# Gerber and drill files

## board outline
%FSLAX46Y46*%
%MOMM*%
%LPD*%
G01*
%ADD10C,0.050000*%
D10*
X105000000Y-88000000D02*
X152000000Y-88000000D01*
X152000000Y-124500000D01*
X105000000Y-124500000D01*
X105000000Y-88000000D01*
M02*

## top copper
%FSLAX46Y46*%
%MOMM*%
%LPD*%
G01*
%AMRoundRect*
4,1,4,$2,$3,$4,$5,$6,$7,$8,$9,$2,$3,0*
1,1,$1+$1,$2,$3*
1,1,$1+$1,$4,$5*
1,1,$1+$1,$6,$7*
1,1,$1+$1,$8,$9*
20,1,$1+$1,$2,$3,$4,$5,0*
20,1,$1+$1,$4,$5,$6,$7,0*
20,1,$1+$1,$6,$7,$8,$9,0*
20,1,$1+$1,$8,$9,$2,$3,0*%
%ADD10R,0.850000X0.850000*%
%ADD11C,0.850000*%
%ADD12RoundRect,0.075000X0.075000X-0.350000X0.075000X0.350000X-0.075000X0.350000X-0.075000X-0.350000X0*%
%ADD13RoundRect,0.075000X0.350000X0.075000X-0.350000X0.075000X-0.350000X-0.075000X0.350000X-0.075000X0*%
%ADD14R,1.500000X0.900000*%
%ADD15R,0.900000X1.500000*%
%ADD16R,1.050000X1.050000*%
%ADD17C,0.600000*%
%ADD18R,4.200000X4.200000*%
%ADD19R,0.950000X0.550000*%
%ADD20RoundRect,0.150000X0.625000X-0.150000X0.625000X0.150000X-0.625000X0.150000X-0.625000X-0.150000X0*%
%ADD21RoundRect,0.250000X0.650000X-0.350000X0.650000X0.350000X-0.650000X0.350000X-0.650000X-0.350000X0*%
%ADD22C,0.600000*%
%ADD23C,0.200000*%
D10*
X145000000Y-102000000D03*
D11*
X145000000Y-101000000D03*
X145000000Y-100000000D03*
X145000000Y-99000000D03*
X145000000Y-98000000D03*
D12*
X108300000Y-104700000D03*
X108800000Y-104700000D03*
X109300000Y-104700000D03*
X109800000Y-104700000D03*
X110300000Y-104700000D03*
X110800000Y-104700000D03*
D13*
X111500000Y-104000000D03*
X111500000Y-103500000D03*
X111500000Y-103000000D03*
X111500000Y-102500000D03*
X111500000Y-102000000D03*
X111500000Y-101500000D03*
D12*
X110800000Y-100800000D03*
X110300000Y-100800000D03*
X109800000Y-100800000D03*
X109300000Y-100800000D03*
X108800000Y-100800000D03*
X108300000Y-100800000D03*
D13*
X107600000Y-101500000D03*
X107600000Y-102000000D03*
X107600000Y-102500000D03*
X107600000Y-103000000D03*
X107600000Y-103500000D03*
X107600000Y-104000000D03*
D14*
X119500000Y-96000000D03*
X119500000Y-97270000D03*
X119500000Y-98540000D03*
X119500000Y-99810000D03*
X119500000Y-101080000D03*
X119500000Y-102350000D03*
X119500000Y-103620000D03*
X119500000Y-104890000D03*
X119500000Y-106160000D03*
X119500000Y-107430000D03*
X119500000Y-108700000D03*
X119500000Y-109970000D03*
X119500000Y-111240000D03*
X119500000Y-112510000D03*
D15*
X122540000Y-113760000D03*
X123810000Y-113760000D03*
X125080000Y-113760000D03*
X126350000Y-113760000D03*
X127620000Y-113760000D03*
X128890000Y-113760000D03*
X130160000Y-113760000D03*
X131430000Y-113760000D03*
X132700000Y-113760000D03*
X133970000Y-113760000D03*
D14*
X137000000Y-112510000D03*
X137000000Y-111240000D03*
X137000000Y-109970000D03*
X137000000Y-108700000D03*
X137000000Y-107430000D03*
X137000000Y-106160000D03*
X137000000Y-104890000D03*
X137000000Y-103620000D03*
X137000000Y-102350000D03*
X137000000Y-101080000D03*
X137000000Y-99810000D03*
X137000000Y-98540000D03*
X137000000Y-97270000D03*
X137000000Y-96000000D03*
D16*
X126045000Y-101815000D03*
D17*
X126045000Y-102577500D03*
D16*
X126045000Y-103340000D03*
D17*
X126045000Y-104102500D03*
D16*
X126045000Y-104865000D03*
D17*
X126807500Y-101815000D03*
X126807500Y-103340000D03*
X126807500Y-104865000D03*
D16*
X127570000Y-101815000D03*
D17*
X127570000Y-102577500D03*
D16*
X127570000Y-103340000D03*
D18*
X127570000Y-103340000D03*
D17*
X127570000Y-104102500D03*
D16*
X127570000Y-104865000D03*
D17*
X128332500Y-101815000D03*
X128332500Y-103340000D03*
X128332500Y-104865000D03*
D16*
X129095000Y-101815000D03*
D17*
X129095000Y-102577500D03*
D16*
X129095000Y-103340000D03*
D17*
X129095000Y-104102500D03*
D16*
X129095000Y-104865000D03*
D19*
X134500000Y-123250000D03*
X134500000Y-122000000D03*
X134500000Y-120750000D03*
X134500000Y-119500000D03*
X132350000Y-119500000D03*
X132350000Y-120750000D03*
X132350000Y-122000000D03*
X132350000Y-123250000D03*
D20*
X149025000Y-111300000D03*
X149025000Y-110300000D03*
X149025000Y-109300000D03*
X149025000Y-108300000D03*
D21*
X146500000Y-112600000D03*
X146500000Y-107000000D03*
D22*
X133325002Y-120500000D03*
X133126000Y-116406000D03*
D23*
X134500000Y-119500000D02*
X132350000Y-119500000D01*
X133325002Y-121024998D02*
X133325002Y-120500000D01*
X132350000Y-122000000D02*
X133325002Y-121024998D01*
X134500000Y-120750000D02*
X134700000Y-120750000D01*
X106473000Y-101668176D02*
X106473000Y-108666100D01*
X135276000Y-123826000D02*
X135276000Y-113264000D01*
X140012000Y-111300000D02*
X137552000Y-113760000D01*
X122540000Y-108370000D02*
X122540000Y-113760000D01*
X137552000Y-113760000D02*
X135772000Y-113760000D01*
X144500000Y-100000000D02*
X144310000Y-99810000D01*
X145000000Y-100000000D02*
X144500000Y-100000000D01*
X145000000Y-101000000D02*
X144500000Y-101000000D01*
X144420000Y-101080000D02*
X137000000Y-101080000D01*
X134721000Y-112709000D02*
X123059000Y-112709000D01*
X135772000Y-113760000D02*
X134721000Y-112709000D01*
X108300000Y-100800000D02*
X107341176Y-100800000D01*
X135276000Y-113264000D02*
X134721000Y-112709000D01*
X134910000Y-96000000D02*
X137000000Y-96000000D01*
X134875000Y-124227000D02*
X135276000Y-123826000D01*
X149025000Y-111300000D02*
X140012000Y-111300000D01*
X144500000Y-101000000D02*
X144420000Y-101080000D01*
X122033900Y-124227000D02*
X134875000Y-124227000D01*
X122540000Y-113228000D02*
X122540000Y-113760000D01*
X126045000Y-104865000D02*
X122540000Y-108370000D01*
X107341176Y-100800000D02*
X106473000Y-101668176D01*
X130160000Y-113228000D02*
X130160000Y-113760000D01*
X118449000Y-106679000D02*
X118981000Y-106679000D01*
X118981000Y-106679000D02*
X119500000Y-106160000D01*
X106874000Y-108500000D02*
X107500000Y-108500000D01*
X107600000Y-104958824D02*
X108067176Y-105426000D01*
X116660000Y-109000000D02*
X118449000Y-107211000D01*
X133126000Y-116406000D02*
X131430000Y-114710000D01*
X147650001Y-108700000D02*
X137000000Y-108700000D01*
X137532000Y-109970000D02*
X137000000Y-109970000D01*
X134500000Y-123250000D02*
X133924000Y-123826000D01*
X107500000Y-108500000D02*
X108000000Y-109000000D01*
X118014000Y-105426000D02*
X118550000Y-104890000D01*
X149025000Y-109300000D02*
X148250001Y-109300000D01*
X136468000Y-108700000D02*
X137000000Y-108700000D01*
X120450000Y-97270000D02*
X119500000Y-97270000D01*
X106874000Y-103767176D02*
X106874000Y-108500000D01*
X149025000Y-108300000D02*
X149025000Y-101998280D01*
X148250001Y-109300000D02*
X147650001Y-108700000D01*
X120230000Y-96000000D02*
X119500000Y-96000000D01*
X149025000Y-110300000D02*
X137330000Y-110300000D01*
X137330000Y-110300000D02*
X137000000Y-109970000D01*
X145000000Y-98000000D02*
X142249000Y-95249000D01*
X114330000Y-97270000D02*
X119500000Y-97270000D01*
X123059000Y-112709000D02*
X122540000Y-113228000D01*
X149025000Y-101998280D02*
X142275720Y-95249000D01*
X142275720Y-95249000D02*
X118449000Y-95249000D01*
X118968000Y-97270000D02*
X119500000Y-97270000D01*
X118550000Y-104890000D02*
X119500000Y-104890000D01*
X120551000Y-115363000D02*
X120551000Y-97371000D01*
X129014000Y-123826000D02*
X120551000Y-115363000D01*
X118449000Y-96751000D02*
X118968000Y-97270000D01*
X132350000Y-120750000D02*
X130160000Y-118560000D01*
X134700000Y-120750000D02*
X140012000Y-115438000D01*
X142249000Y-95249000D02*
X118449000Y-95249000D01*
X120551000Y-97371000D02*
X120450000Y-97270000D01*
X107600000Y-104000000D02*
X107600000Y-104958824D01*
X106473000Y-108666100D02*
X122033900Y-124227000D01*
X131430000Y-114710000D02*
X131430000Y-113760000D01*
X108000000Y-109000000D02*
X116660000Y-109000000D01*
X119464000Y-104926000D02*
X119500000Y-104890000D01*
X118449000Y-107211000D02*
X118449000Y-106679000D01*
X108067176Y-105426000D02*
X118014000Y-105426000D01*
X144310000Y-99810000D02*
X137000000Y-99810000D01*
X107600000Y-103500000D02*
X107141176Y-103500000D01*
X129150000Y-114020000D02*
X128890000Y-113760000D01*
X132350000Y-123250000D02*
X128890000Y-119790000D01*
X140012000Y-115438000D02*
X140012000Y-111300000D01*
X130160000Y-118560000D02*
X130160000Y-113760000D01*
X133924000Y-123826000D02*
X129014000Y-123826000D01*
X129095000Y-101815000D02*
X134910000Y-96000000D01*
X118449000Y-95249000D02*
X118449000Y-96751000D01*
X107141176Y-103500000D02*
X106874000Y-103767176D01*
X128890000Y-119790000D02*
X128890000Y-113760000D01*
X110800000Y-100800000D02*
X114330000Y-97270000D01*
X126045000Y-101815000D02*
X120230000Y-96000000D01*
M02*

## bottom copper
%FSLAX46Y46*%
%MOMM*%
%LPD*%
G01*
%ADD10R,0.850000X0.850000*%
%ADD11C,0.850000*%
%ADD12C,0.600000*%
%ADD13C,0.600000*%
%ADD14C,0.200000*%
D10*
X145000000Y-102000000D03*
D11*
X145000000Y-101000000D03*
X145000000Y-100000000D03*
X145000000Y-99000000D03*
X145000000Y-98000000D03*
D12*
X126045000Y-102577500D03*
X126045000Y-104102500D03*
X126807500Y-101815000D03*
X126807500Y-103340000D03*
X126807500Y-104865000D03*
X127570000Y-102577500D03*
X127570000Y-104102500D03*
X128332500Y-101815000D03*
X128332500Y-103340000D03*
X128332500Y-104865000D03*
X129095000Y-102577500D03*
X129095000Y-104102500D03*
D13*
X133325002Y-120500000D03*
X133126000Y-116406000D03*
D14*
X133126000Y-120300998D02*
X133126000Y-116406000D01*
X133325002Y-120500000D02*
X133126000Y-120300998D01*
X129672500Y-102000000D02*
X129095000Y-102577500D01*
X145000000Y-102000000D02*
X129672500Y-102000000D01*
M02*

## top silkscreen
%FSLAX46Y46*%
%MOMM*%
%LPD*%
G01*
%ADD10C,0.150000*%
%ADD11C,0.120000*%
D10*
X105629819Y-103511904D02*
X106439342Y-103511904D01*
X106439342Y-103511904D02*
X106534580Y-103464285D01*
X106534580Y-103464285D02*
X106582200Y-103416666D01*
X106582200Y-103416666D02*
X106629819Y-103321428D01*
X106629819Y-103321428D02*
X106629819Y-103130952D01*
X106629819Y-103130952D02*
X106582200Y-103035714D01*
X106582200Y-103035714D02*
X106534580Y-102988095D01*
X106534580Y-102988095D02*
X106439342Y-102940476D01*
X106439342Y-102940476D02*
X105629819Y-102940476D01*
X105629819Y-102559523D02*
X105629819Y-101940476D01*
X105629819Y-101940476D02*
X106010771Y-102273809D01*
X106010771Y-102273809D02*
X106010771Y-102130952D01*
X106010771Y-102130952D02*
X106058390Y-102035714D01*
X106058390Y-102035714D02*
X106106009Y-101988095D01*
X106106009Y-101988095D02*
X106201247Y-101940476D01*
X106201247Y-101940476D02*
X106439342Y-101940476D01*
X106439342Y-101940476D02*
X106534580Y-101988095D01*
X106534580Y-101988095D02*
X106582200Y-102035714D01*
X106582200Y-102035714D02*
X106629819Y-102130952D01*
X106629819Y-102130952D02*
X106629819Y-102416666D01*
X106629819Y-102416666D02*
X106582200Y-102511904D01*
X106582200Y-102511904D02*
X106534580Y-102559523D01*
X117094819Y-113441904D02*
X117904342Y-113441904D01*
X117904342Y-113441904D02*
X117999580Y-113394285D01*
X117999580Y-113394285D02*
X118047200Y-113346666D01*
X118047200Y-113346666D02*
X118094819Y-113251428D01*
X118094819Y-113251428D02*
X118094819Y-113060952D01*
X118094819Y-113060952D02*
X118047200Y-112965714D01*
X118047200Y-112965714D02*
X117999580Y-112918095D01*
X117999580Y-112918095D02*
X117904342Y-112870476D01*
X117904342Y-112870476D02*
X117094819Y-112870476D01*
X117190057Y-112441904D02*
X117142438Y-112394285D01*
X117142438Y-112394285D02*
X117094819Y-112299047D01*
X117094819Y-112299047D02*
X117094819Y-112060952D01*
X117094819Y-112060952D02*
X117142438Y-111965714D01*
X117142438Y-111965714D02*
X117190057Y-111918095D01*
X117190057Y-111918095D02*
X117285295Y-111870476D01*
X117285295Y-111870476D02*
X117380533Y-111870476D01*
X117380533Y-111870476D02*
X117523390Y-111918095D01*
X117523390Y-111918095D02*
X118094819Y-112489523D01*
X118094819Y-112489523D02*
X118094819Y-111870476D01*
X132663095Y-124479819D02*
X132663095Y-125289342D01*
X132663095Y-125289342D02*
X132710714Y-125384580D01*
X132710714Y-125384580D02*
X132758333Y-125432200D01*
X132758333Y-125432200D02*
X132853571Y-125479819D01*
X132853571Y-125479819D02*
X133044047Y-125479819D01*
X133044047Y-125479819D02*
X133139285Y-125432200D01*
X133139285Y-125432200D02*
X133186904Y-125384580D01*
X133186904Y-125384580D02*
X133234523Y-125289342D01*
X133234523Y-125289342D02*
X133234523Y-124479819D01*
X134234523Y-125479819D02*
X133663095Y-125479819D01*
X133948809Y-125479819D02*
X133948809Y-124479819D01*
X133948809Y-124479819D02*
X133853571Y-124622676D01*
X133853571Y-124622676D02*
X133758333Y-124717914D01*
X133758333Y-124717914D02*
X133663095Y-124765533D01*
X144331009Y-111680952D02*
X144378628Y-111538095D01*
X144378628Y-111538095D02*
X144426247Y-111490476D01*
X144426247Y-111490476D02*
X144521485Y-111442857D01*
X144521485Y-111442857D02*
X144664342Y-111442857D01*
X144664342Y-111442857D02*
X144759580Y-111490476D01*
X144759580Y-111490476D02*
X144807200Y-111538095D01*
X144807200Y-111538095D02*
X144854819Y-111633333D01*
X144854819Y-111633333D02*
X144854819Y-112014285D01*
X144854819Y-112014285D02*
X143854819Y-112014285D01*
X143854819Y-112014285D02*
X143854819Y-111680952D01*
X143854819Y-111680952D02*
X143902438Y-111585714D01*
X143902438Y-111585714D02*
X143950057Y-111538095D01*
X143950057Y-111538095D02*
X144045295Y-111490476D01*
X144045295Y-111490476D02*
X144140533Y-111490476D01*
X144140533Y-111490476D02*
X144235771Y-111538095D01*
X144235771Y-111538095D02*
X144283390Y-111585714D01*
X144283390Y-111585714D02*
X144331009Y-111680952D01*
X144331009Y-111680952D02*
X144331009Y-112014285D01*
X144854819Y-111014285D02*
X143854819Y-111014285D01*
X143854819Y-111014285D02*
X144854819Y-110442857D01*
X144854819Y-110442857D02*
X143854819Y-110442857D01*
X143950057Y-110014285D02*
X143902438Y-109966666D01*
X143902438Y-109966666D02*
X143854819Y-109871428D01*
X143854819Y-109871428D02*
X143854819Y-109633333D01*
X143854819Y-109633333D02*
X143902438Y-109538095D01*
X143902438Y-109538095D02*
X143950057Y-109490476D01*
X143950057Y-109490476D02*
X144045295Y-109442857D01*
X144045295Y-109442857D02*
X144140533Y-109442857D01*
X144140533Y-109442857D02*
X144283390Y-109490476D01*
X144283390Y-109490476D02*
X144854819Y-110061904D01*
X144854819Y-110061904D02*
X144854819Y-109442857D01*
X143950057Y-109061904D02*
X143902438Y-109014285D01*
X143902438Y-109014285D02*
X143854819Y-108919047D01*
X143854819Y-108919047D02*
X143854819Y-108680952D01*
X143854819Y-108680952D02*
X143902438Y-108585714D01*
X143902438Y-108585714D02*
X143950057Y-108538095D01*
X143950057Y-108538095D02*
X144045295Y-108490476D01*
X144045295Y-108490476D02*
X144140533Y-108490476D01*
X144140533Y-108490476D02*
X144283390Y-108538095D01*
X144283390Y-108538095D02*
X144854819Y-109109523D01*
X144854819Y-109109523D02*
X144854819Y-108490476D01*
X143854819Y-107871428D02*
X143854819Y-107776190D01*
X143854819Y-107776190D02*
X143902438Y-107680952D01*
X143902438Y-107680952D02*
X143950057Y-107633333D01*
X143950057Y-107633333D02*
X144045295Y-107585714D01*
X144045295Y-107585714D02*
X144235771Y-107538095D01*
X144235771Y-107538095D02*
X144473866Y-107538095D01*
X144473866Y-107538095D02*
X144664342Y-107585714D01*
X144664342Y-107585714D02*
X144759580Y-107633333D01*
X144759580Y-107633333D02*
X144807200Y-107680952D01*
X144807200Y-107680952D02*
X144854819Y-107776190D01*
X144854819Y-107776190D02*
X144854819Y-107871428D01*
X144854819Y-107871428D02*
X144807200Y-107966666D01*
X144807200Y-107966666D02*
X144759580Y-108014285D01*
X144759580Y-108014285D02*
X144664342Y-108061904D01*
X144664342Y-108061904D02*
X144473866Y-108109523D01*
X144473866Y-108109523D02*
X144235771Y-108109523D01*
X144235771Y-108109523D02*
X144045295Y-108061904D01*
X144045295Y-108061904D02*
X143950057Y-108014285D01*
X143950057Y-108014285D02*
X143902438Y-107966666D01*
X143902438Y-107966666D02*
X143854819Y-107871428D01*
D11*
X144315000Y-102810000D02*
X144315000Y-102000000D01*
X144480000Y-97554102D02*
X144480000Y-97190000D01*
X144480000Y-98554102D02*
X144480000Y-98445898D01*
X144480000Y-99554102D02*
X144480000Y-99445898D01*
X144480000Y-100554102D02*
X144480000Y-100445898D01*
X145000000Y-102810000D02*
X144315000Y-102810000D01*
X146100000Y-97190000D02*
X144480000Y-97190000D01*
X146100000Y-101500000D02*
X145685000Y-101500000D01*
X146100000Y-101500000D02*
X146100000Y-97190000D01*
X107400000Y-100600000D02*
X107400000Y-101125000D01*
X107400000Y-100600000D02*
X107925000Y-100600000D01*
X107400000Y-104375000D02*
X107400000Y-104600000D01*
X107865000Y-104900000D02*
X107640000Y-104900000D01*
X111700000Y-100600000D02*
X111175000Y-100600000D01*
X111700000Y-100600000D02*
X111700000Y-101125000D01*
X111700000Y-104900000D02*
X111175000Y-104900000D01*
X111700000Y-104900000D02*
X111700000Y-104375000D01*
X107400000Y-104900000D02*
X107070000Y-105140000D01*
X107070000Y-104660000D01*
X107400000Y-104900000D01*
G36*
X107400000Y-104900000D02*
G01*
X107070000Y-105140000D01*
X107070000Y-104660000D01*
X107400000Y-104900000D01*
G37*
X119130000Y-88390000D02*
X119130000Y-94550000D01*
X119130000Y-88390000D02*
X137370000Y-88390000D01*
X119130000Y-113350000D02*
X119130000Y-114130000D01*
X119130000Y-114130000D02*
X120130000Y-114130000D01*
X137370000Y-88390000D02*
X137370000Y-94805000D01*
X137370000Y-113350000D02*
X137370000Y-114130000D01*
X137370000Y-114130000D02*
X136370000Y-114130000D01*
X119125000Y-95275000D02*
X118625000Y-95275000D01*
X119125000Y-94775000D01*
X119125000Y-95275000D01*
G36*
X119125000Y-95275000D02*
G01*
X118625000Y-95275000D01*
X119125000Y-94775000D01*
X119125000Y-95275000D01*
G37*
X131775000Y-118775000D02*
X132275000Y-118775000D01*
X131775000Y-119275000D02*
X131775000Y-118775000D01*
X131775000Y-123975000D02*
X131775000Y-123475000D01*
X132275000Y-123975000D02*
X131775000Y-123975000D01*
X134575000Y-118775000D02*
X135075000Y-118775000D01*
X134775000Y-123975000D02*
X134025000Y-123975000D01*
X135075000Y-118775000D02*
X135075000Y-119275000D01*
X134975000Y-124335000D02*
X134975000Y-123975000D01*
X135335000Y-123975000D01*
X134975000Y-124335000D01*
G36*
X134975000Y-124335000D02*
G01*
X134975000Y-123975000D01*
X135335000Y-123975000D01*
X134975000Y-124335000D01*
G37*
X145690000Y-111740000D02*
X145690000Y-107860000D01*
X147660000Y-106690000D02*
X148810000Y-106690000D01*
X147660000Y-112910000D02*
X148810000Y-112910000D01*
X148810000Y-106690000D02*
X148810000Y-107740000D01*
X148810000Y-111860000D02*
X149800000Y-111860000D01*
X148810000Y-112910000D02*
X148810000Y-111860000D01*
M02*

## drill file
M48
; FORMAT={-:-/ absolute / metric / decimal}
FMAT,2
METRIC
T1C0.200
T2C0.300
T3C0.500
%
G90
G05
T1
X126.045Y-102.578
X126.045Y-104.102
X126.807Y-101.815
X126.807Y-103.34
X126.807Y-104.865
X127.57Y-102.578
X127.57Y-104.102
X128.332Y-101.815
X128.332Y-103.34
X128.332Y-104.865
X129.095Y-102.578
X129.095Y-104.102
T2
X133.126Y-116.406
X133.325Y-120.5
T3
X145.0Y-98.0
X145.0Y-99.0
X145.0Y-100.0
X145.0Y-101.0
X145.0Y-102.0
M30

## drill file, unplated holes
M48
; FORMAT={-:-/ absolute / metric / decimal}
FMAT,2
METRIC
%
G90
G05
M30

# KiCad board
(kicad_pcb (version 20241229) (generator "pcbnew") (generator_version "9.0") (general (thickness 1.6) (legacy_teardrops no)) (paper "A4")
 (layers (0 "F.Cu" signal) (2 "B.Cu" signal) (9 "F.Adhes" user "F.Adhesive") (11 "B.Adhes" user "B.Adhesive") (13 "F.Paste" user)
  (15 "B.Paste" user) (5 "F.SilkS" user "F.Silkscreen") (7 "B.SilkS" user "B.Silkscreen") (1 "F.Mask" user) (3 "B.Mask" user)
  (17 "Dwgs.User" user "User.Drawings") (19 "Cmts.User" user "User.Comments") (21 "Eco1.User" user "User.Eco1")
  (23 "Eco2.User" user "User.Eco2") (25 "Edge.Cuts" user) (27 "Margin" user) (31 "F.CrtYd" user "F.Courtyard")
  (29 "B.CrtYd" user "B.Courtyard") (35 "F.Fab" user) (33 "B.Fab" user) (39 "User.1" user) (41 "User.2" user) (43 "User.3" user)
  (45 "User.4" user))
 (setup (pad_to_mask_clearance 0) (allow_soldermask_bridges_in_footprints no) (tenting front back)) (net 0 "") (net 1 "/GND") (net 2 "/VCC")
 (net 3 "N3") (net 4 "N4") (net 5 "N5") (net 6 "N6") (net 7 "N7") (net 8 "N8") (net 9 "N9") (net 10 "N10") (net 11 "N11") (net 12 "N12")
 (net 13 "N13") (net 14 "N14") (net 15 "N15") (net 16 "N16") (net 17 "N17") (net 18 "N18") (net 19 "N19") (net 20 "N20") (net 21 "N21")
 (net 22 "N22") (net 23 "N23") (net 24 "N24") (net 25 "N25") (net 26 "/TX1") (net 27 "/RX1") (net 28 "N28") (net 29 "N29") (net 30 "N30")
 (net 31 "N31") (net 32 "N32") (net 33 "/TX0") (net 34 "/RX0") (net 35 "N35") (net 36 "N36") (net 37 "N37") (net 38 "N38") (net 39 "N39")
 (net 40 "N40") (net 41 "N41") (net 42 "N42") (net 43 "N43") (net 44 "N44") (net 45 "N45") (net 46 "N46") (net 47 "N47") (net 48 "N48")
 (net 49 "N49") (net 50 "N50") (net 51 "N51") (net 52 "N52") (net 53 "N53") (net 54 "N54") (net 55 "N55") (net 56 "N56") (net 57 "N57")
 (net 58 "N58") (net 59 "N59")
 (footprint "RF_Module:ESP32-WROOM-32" (layer "F.Cu") (at 128.25 104.25)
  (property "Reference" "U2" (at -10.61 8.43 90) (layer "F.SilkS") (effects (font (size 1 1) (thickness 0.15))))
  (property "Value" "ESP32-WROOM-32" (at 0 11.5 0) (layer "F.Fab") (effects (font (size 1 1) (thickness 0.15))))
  (fp_line (start -9.12 -15.86) (end -9.12 -9.7) (stroke (width 0.12) (type solid)) (layer "F.SilkS"))
  (fp_line (start -9.12 -15.86) (end 9.12 -15.86) (stroke (width 0.12) (type solid)) (layer "F.SilkS"))
  (fp_line (start -9.12 9.1) (end -9.12 9.88) (stroke (width 0.12) (type solid)) (layer "F.SilkS"))
  (fp_line (start -9.12 9.88) (end -8.12 9.88) (stroke (width 0.12) (type solid)) (layer "F.SilkS"))
  (fp_line (start 9.12 -15.86) (end 9.12 -9.445) (stroke (width 0.12) (type solid)) (layer "F.SilkS"))
  (fp_line (start 9.12 9.1) (end 9.12 9.88) (stroke (width 0.12) (type solid)) (layer "F.SilkS"))
  (fp_line (start 9.12 9.88) (end 8.12 9.88) (stroke (width 0.12) (type solid)) (layer "F.SilkS"))
  (fp_poly
   (pts (xy -9.125 -8.975) (xy -9.625 -8.975) (xy -9.125 -9.475) (xy -9.125 -8.975)) (stroke (width 0.12) (type solid)) (fill yes)
   (layer "F.SilkS"))
  (pad "1" smd rect (at -8.75 -8.25) (size 1.5 0.9) (layers "F.Cu" "F.Mask" "F.Paste") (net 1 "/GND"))
  (pad "2" smd rect (at -8.75 -6.98) (size 1.5 0.9) (layers "F.Cu" "F.Mask" "F.Paste") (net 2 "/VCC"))
  (pad "3" smd rect (at -8.75 -5.71) (size 1.5 0.9) (layers "F.Cu" "F.Mask" "F.Paste") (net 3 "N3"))
  (pad "4" smd rect (at -8.75 -4.44) (size 1.5 0.9) (layers "F.Cu" "F.Mask" "F.Paste") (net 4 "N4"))
  (pad "5" smd rect (at -8.75 -3.17) (size 1.5 0.9) (layers "F.Cu" "F.Mask" "F.Paste") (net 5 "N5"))
  (pad "6" smd rect (at -8.75 -1.9) (size 1.5 0.9) (layers "F.Cu" "F.Mask" "F.Paste") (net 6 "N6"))
  (pad "7" smd rect (at -8.75 -0.63) (size 1.5 0.9) (layers "F.Cu" "F.Mask" "F.Paste") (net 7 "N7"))
  (pad "8" smd rect (at -8.75 0.64) (size 1.5 0.9) (layers "F.Cu" "F.Mask" "F.Paste") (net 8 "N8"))
  (pad "9" smd rect (at -8.75 1.91) (size 1.5 0.9) (layers "F.Cu" "F.Mask" "F.Paste") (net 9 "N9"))
  (pad "10" smd rect (at -8.75 3.18) (size 1.5 0.9) (layers "F.Cu" "F.Mask" "F.Paste") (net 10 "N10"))
  (pad "11" smd rect (at -8.75 4.45) (size 1.5 0.9) (layers "F.Cu" "F.Mask" "F.Paste") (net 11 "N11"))
  (pad "12" smd rect (at -8.75 5.72) (size 1.5 0.9) (layers "F.Cu" "F.Mask" "F.Paste") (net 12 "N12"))
  (pad "13" smd rect (at -8.75 6.99) (size 1.5 0.9) (layers "F.Cu" "F.Mask" "F.Paste") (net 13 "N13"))
  (pad "14" smd rect (at -8.75 8.26) (size 1.5 0.9) (layers "F.Cu" "F.Mask" "F.Paste") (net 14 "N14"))
  (pad "15" smd rect (at -5.71 9.51 90) (size 1.5 0.9) (layers "F.Cu" "F.Mask" "F.Paste") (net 1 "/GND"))
  (pad "16" smd rect (at -4.44 9.51 90) (size 1.5 0.9) (layers "F.Cu" "F.Mask" "F.Paste") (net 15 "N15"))
  (pad "17" smd rect (at -3.17 9.51 90) (size 1.5 0.9) (layers "F.Cu" "F.Mask" "F.Paste") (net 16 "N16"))
  (pad "18" smd rect (at -1.9 9.51 90) (size 1.5 0.9) (layers "F.Cu" "F.Mask" "F.Paste") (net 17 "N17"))
  (pad "19" smd rect (at -0.63 9.51 90) (size 1.5 0.9) (layers "F.Cu" "F.Mask" "F.Paste") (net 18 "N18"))
  (pad "20" smd rect (at 0.64 9.51 90) (size 1.5 0.9) (layers "F.Cu" "F.Mask" "F.Paste") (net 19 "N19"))
  (pad "21" smd rect (at 1.91 9.51 90) (size 1.5 0.9) (layers "F.Cu" "F.Mask" "F.Paste") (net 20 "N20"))
  (pad "22" smd rect (at 3.18 9.51 90) (size 1.5 0.9) (layers "F.Cu" "F.Mask" "F.Paste") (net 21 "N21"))
  (pad "23" smd rect (at 4.45 9.51 90) (size 1.5 0.9) (layers "F.Cu" "F.Mask" "F.Paste") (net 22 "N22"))
  (pad "24" smd rect (at 5.72 9.51 90) (size 1.5 0.9) (layers "F.Cu" "F.Mask" "F.Paste") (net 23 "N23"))
  (pad "25" smd rect (at 8.75 8.26) (size 1.5 0.9) (layers "F.Cu" "F.Mask" "F.Paste") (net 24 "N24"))
  (pad "26" smd rect (at 8.75 6.99) (size 1.5 0.9) (layers "F.Cu" "F.Mask" "F.Paste") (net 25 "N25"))
  (pad "27" smd rect (at 8.75 5.72) (size 1.5 0.9) (layers "F.Cu" "F.Mask" "F.Paste") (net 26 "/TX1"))
  (pad "28" smd rect (at 8.75 4.45) (size 1.5 0.9) (layers "F.Cu" "F.Mask" "F.Paste") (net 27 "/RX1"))
  (pad "29" smd rect (at 8.75 3.18) (size 1.5 0.9) (layers "F.Cu" "F.Mask" "F.Paste") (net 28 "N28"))
  (pad "30" smd rect (at 8.75 1.91) (size 1.5 0.9) (layers "F.Cu" "F.Mask" "F.Paste") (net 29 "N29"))
  (pad "31" smd rect (at 8.75 0.64) (size 1.5 0.9) (layers "F.Cu" "F.Mask" "F.Paste") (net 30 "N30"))
  (pad "32" smd rect (at 8.75 -0.63) (size 1.5 0.9) (layers "F.Cu" "F.Mask" "F.Paste") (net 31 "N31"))
  (pad "33" smd rect (at 8.75 -1.9) (size 1.5 0.9) (layers "F.Cu" "F.Mask" "F.Paste") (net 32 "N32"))
  (pad "34" smd rect (at 8.75 -3.17) (size 1.5 0.9) (layers "F.Cu" "F.Mask" "F.Paste") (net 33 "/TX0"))
  (pad "35" smd rect (at 8.75 -4.44) (size 1.5 0.9) (layers "F.Cu" "F.Mask" "F.Paste") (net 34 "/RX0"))
  (pad "36" smd rect (at 8.75 -5.71) (size 1.5 0.9) (layers "F.Cu" "F.Mask" "F.Paste") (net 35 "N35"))
  (pad "37" smd rect (at 8.75 -6.98) (size 1.5 0.9) (layers "F.Cu" "F.Mask" "F.Paste") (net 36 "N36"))
  (pad "38" smd rect (at 8.75 -8.25) (size 1.5 0.9) (layers "F.Cu" "F.Mask" "F.Paste") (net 1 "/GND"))
  (pad "39" smd rect (at -2.205 -2.435) (size 1.05 1.05) (layers "F.Cu" "F.Paste") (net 1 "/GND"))
  (pad "39" thru_hole circle (at -2.205 -1.6725) (size 0.6 0.6) (drill 0.2) (layers "*.Cu" "F.Mask") (remove_unused_layers no)
   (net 1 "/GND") (zone_connect 2))
  (pad "39" smd rect (at -2.205 -0.91) (size 1.05 1.05) (layers "F.Cu" "F.Paste") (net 1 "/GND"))
  (pad "39" thru_hole circle (at -2.205 -0.1475) (size 0.6 0.6) (drill 0.2) (layers "*.Cu" "F.Mask") (remove_unused_layers no)
   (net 1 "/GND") (zone_connect 2))
  (pad "39" smd rect (at -2.205 0.615) (size 1.05 1.05) (layers "F.Cu" "F.Paste") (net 1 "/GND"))
  (pad "39" thru_hole circle (at -1.4425 -2.435) (size 0.6 0.6) (drill 0.2) (layers "*.Cu" "F.Mask") (remove_unused_layers no)
   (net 1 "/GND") (zone_connect 2))
  (pad "39" thru_hole circle (at -1.4425 -0.91) (size 0.6 0.6) (drill 0.2) (layers "*.Cu" "F.Mask") (remove_unused_layers no) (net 1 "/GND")
   (zone_connect 2))
  (pad "39" thru_hole circle (at -1.4425 0.615) (size 0.6 0.6) (drill 0.2) (layers "*.Cu" "F.Mask") (remove_unused_layers no) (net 1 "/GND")
   (zone_connect 2))
  (pad "39" smd rect (at -0.68 -2.435) (size 1.05 1.05) (layers "F.Cu" "F.Paste") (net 1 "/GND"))
  (pad "39" thru_hole circle (at -0.68 -1.6725) (size 0.6 0.6) (drill 0.2) (layers "*.Cu" "F.Mask") (remove_unused_layers no) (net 1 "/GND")
   (zone_connect 2))
  (pad "39" smd rect (at -0.68 -0.91) (size 1.05 1.05) (layers "F.Cu" "F.Paste") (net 1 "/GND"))
  (pad "39" smd rect (at -0.68 -0.91) (size 4.2 4.2) (layers "F.Cu" "F.Mask") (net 1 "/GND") (zone_connect 2))
  (pad "39" thru_hole circle (at -0.68 -0.1475) (size 0.6 0.6) (drill 0.2) (layers "*.Cu" "F.Mask") (remove_unused_layers no) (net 1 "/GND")
   (zone_connect 2))
  (pad "39" smd rect (at -0.68 0.615) (size 1.05 1.05) (layers "F.Cu" "F.Paste") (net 1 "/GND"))
  (pad "39" thru_hole circle (at 0.0825 -2.435) (size 0.6 0.6) (drill 0.2) (layers "*.Cu" "F.Mask") (remove_unused_layers no) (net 1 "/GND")
   (zone_connect 2))
  (pad "39" thru_hole circle (at 0.0825 -0.91) (size 0.6 0.6) (drill 0.2) (layers "*.Cu" "F.Mask") (remove_unused_layers no) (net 1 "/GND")
   (zone_connect 2))
  (pad "39" thru_hole circle (at 0.0825 0.615) (size 0.6 0.6) (drill 0.2) (layers "*.Cu" "F.Mask") (remove_unused_layers no) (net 1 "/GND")
   (zone_connect 2))
  (pad "39" smd rect (at 0.845 -2.435) (size 1.05 1.05) (layers "F.Cu" "F.Paste") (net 1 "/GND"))
  (pad "39" thru_hole circle (at 0.845 -1.6725) (size 0.6 0.6) (drill 0.2) (layers "*.Cu" "F.Mask") (remove_unused_layers no) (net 1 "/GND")
   (zone_connect 2))
  (pad "39" smd rect (at 0.845 -0.91) (size 1.05 1.05) (layers "F.Cu" "F.Paste") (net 1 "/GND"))
  (pad "39" thru_hole circle (at 0.845 -0.1475) (size 0.6 0.6) (drill 0.2) (layers "*.Cu" "F.Mask") (remove_unused_layers no) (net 1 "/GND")
   (zone_connect 2))
  (pad "39" smd rect (at 0.845 0.615) (size 1.05 1.05) (layers "F.Cu" "F.Paste") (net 1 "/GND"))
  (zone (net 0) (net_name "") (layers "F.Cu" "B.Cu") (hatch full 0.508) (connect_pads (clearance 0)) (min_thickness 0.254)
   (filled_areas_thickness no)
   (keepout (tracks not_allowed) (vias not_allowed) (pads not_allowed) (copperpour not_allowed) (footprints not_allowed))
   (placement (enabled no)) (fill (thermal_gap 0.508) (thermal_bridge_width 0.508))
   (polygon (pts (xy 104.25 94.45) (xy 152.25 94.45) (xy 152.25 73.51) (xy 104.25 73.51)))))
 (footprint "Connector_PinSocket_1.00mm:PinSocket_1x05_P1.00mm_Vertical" (layer "F.Cu") (at 145 102 180)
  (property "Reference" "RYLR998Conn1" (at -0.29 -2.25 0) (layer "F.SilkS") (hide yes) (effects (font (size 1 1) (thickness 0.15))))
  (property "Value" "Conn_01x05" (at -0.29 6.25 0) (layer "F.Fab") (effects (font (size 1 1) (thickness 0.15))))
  (fp_line (start 0.685 -0.81) (end 0.685 0) (stroke (width 0.12) (type solid)) (layer "F.SilkS"))
  (fp_line (start 0.52 4.445898) (end 0.52 4.81) (stroke (width 0.12) (type solid)) (layer "F.SilkS"))
  (fp_line (start 0.52 3.445898) (end 0.52 3.554102) (stroke (width 0.12) (type solid)) (layer "F.SilkS"))
  (fp_line (start 0.52 2.445898) (end 0.52 2.554102) (stroke (width 0.12) (type solid)) (layer "F.SilkS"))
  (fp_line (start 0.52 1.445898) (end 0.52 1.554102) (stroke (width 0.12) (type solid)) (layer "F.SilkS"))
  (fp_line (start 0 -0.81) (end 0.685 -0.81) (stroke (width 0.12) (type solid)) (layer "F.SilkS"))
  (fp_line (start -1.1 4.81) (end 0.52 4.81) (stroke (width 0.12) (type solid)) (layer "F.SilkS"))
  (fp_line (start -1.1 0.5) (end -0.685 0.5) (stroke (width 0.12) (type solid)) (layer "F.SilkS"))
  (fp_line (start -1.1 0.5) (end -1.1 4.81) (stroke (width 0.12) (type solid)) (layer "F.SilkS"))
  (pad "1" thru_hole rect (at 0 0 180) (size 0.85 0.85) (drill 0.5) (layers "*.Cu" "*.Mask") (remove_unused_layers no) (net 1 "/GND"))
  (pad "2" thru_hole circle (at 0 1 180) (size 0.85 0.85) (drill 0.5) (layers "*.Cu" "*.Mask") (remove_unused_layers no) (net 33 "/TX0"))
  (pad "3" thru_hole circle (at 0 2 180) (size 0.85 0.85) (drill 0.5) (layers "*.Cu" "*.Mask") (remove_unused_layers no) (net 34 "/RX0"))
  (pad "4" thru_hole circle (at 0 3 180) (size 0.85 0.85) (drill 0.5) (layers "*.Cu" "*.Mask") (remove_unused_layers no) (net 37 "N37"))
  (pad "5" thru_hole circle (at 0 4 180) (size 0.85 0.85) (drill 0.5) (layers "*.Cu" "*.Mask") (remove_unused_layers no) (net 2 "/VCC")))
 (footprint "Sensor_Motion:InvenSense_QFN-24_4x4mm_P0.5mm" (layer "F.Cu") (at 109.55 102.75 90)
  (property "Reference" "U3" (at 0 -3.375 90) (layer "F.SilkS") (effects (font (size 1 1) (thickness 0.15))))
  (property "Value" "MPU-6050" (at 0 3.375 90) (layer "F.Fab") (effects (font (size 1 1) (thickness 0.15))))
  (fp_line (start 2.15 -2.15) (end 1.625 -2.15) (stroke (width 0.12) (type solid)) (layer "F.SilkS"))
  (fp_line (start 2.15 -2.15) (end 2.15 -1.625) (stroke (width 0.12) (type solid)) (layer "F.SilkS"))
  (fp_line (start -1.625 -2.15) (end -1.85 -2.15) (stroke (width 0.12) (type solid)) (layer "F.SilkS"))
  (fp_line (start -2.15 -1.685) (end -2.15 -1.91) (stroke (width 0.12) (type solid)) (layer "F.SilkS"))
  (fp_line (start 2.15 2.15) (end 2.15 1.625) (stroke (width 0.12) (type solid)) (layer "F.SilkS"))
  (fp_line (start 2.15 2.15) (end 1.625 2.15) (stroke (width 0.12) (type solid)) (layer "F.SilkS"))
  (fp_line (start -2.15 2.15) (end -2.15 1.625) (stroke (width 0.12) (type solid)) (layer "F.SilkS"))
  (fp_line (start -2.15 2.15) (end -1.625 2.15) (stroke (width 0.12) (type solid)) (layer "F.SilkS"))
  (fp_poly
   (pts (xy -2.15 -2.15) (xy -2.39 -2.48) (xy -1.91 -2.48) (xy -2.15 -2.15)) (stroke (width 0.12) (type solid)) (fill yes) (layer "F.SilkS"))
  (pad "1" smd roundrect (at -1.95 -1.25 90) (size 0.85 0.3) (layers "F.Cu" "F.Mask" "F.Paste") (roundrect_rratio 0.25) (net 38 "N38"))
  (pad "2" smd roundrect (at -1.95 -0.75 90) (size 0.85 0.3) (layers "F.Cu" "F.Mask" "F.Paste") (roundrect_rratio 0.25) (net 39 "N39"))
  (pad "3" smd roundrect (at -1.95 -0.25 90) (size 0.85 0.3) (layers "F.Cu" "F.Mask" "F.Paste") (roundrect_rratio 0.25) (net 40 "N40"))
  (pad "4" smd roundrect (at -1.95 0.25 90) (size 0.85 0.3) (layers "F.Cu" "F.Mask" "F.Paste") (roundrect_rratio 0.25) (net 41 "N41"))
  (pad "5" smd roundrect (at -1.95 0.75 90) (size 0.85 0.3) (layers "F.Cu" "F.Mask" "F.Paste") (roundrect_rratio 0.25) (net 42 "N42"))
  (pad "6" smd roundrect (at -1.95 1.25 90) (size 0.85 0.3) (layers "F.Cu" "F.Mask" "F.Paste") (roundrect_rratio 0.25) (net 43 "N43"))
  (pad "7" smd roundrect (at -1.25 1.95 180) (size 0.85 0.3) (layers "F.Cu" "F.Mask" "F.Paste") (roundrect_rratio 0.25) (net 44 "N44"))
  (pad "8" smd roundrect (at -0.75 1.95 180) (size 0.85 0.3) (layers "F.Cu" "F.Mask" "F.Paste") (roundrect_rratio 0.25) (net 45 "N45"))
  (pad "9" smd roundrect (at -0.25 1.95 180) (size 0.85 0.3) (layers "F.Cu" "F.Mask" "F.Paste") (roundrect_rratio 0.25) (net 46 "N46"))
  (pad "10" smd roundrect (at 0.25 1.95 180) (size 0.85 0.3) (layers "F.Cu" "F.Mask" "F.Paste") (roundrect_rratio 0.25) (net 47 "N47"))
  (pad "11" smd roundrect (at 0.75 1.95 180) (size 0.85 0.3) (layers "F.Cu" "F.Mask" "F.Paste") (roundrect_rratio 0.25) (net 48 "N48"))
  (pad "12" smd roundrect (at 1.25 1.95 180) (size 0.85 0.3) (layers "F.Cu" "F.Mask" "F.Paste") (roundrect_rratio 0.25) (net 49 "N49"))
  (pad "13" smd roundrect (at 1.95 1.25 90) (size 0.85 0.3) (layers "F.Cu" "F.Mask" "F.Paste") (roundrect_rratio 0.25) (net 2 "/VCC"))
  (pad "14" smd roundrect (at 1.95 0.75 90) (size 0.85 0.3) (layers "F.Cu" "F.Mask" "F.Paste") (roundrect_rratio 0.25) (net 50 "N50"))
  (pad "15" smd roundrect (at 1.95 0.25 90) (size 0.85 0.3) (layers "F.Cu" "F.Mask" "F.Paste") (roundrect_rratio 0.25) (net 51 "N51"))
  (pad "16" smd roundrect (at 1.95 -0.25 90) (size 0.85 0.3) (layers "F.Cu" "F.Mask" "F.Paste") (roundrect_rratio 0.25) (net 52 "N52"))
  (pad "17" smd roundrect (at 1.95 -0.75 90) (size 0.85 0.3) (layers "F.Cu" "F.Mask" "F.Paste") (roundrect_rratio 0.25) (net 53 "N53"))
  (pad "18" smd roundrect (at 1.95 -1.25 90) (size 0.85 0.3) (layers "F.Cu" "F.Mask" "F.Paste") (roundrect_rratio 0.25) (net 1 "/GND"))
  (pad "19" smd roundrect (at 1.25 -1.95 180) (size 0.85 0.3) (layers "F.Cu" "F.Mask" "F.Paste") (roundrect_rratio 0.25) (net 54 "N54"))
  (pad "20" smd roundrect (at 0.75 -1.95 180) (size 0.85 0.3) (layers "F.Cu" "F.Mask" "F.Paste") (roundrect_rratio 0.25) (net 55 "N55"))
  (pad "21" smd roundrect (at 0.25 -1.95 180) (size 0.85 0.3) (layers "F.Cu" "F.Mask" "F.Paste") (roundrect_rratio 0.25) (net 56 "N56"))
  (pad "22" smd roundrect (at -0.25 -1.95 180) (size 0.85 0.3) (layers "F.Cu" "F.Mask" "F.Paste") (roundrect_rratio 0.25) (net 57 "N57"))
  (pad "23" smd roundrect (at -0.75 -1.95 180) (size 0.85 0.3) (layers "F.Cu" "F.Mask" "F.Paste") (roundrect_rratio 0.25) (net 9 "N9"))
  (pad "24" smd roundrect (at -1.25 -1.95 180) (size 0.85 0.3) (layers "F.Cu" "F.Mask" "F.Paste") (roundrect_rratio 0.25) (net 8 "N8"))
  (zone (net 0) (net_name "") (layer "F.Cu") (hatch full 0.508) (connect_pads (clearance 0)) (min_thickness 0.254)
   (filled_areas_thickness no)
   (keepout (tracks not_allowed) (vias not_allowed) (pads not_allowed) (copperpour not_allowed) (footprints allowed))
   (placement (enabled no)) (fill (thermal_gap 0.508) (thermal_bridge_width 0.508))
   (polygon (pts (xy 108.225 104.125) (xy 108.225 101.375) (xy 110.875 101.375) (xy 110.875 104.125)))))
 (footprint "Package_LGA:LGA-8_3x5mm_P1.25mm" (layer "F.Cu") (at 133.425 121.375 180)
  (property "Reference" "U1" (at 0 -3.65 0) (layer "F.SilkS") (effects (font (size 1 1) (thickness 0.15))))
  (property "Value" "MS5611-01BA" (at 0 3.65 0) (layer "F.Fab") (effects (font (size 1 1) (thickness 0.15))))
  (fp_line (start 1.65 2.6) (end 1.15 2.6) (stroke (width 0.12) (type solid)) (layer "F.SilkS"))
  (fp_line (start 1.65 2.1) (end 1.65 2.6) (stroke (width 0.12) (type solid)) (layer "F.SilkS"))
  (fp_line (start 1.65 -2.6) (end 1.65 -2.1) (stroke (width 0.12) (type solid)) (layer "F.SilkS"))
  (fp_line (start 1.15 -2.6) (end 1.65 -2.6) (stroke (width 0.12) (type solid)) (layer "F.SilkS"))
  (fp_line (start -1.15 2.6) (end -1.65 2.6) (stroke (width 0.12) (type solid)) (layer "F.SilkS"))
  (fp_line (start -1.35 -2.6) (end -0.6 -2.6) (stroke (width 0.12) (type solid)) (layer "F.SilkS"))
  (fp_line (start -1.65 2.6) (end -1.65 2.1) (stroke (width 0.12) (type solid)) (layer "F.SilkS"))
  (fp_poly
   (pts (xy -1.55 -2.6) (xy -1.91 -2.6) (xy -1.55 -2.96) (xy -1.55 -2.6)) (stroke (width 0.12) (type solid)) (fill yes) (layer "F.SilkS"))
  (pad "1" smd rect (at -1.075 -1.875 180) (size 0.95 0.55) (layers "F.Cu" "F.Mask" "F.Paste") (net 2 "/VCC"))
  (pad "2" smd rect (at -1.075 -0.625 180) (size 0.95 0.55) (layers "F.Cu" "F.Mask" "F.Paste") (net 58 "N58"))
  (pad "3" smd rect (at -1.075 0.625 180) (size 0.95 0.55) (layers "F.Cu" "F.Mask" "F.Paste") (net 1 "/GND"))
  (pad "4" smd rect (at -1.075 1.875 180) (size 0.95 0.55) (layers "F.Cu" "F.Mask" "F.Paste") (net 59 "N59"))
  (pad "5" smd rect (at 1.075 1.875 180) (size 0.95 0.55) (layers "F.Cu" "F.Mask" "F.Paste") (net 59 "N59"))
  (pad "6" smd rect (at 1.075 0.625 180) (size 0.95 0.55) (layers "F.Cu" "F.Mask" "F.Paste") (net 20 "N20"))
  (pad "7" smd rect (at 1.075 -0.625 180) (size 0.95 0.55) (layers "F.Cu" "F.Mask" "F.Paste") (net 21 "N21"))
  (pad "8" smd rect (at 1.075 -1.875 180) (size 0.95 0.55) (layers "F.Cu" "F.Mask" "F.Paste") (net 19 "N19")))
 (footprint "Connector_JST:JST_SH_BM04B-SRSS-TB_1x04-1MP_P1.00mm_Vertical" (layer "F.Cu") (at 147.7 109.8 90)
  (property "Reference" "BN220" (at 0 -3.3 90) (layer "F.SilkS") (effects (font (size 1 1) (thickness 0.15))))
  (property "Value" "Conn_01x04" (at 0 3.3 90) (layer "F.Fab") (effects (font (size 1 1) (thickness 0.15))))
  (fp_line (start -1.94 -2.01) (end 1.94 -2.01) (stroke (width 0.12) (type solid)) (layer "F.SilkS"))
  (fp_line (start 3.11 -0.04) (end 3.11 1.11) (stroke (width 0.12) (type solid)) (layer "F.SilkS"))
  (fp_line (start -3.11 -0.04) (end -3.11 1.11) (stroke (width 0.12) (type solid)) (layer "F.SilkS"))
  (fp_line (start 3.11 1.11) (end 2.06 1.11) (stroke (width 0.12) (type solid)) (layer "F.SilkS"))
  (fp_line (start -2.06 1.11) (end -2.06 2.1) (stroke (width 0.12) (type solid)) (layer "F.SilkS"))
  (fp_line (start -3.11 1.11) (end -2.06 1.11) (stroke (width 0.12) (type solid)) (layer "F.SilkS"))
  (pad "1" smd roundrect (at -1.5 1.325 90) (size 0.6 1.55) (layers "F.Cu" "F.Mask" "F.Paste") (roundrect_rratio 0.25) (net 1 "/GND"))
  (pad "2" smd roundrect (at -0.5 1.325 90) (size 0.6 1.55) (layers "F.Cu" "F.Mask" "F.Paste") (roundrect_rratio 0.25) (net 26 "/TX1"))
  (pad "3" smd roundrect (at 0.5 1.325 90) (size 0.6 1.55) (layers "F.Cu" "F.Mask" "F.Paste") (roundrect_rratio 0.25) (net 27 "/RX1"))
  (pad "4" smd roundrect (at 1.5 1.325 90) (size 0.6 1.55) (layers "F.Cu" "F.Mask" "F.Paste") (roundrect_rratio 0.25) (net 2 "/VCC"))
  (pad "MP" smd roundrect (at -2.8 -1.2 90) (size 1.2 1.8) (layers "F.Cu" "F.Mask" "F.Paste") (roundrect_rratio 0.208333))
  (pad "MP" smd roundrect (at 2.8 -1.2 90) (size 1.2 1.8) (layers "F.Cu" "F.Mask" "F.Paste") (roundrect_rratio 0.208333)))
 (gr_rect (start 105 88) (end 152 124.5) (stroke (width 0.05) (type default)) (fill no) (layer "Edge.Cuts"))
 (segment (start 132.35 123.25) (end 128.89 119.79) (width 0.2) (layer "F.Cu") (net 19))
 (segment (start 128.89 119.79) (end 128.89 113.76) (width 0.2) (layer "F.Cu") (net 19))
 (segment (start 129.15 114.02) (end 128.89 113.76) (width 0.2) (layer "F.Cu") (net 19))
 (segment (start 134.5 119.5) (end 132.35 119.5) (width 0.2) (layer "F.Cu") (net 59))
 (segment (start 133.325002 121.024998) (end 133.325002 120.5) (width 0.2) (layer "F.Cu") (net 21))
 (segment (start 131.43 114.71) (end 131.43 113.76) (width 0.2) (layer "F.Cu") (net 21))
 (segment (start 132.35 122) (end 133.325002 121.024998) (width 0.2) (layer "F.Cu") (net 21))
 (segment (start 133.126 116.406) (end 131.43 114.71) (width 0.2) (layer "F.Cu") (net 21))
 (via (at 133.126 116.406) (size 0.6) (drill 0.3) (layers "F.Cu" "B.Cu") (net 21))
 (via (at 133.325002 120.5) (size 0.6) (drill 0.3) (layers "F.Cu" "B.Cu") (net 21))
 (segment (start 133.126 120.300998) (end 133.126 116.406) (width 0.2) (layer "B.Cu") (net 21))
 (segment (start 133.325002 120.5) (end 133.126 120.300998) (width 0.2) (layer "B.Cu") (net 21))
 (segment (start 130.16 113.228) (end 130.16 113.76) (width 0.2) (layer "F.Cu") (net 20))
 (segment (start 130.16 118.56) (end 130.16 113.76) (width 0.2) (layer "F.Cu") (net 20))
 (segment (start 132.35 120.75) (end 130.16 118.56) (width 0.2) (layer "F.Cu") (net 20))
 (segment (start 118.981 106.679) (end 119.5 106.16) (width 0.2) (layer "F.Cu") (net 9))
 (segment (start 106.874 108.5) (end 107.5 108.5) (width 0.2) (layer "F.Cu") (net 9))
 (segment (start 116.66 109) (end 118.449 107.211) (width 0.2) (layer "F.Cu") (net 9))
 (segment (start 106.874 103.767176) (end 106.874 108.5) (width 0.2) (layer "F.Cu") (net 9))
 (segment (start 118.449 106.679) (end 118.981 106.679) (width 0.2) (layer "F.Cu") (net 9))
 (segment (start 108 109) (end 116.66 109) (width 0.2) (layer "F.Cu") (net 9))
 (segment (start 107.6 103.5) (end 107.141176 103.5) (width 0.2) (layer "F.Cu") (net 9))
 (segment (start 107.141176 103.5) (end 106.874 103.767176) (width 0.2) (layer "F.Cu") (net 9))
 (segment (start 118.449 107.211) (end 118.449 106.679) (width 0.2) (layer "F.Cu") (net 9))
 (segment (start 107.5 108.5) (end 108 109) (width 0.2) (layer "F.Cu") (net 9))
 (segment (start 118.55 104.89) (end 119.5 104.89) (width 0.2) (layer "F.Cu") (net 8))
 (segment (start 107.6 104) (end 107.6 104.958824) (width 0.2) (layer "F.Cu") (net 8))
 (segment (start 107.6 104.958824) (end 108.067176 105.426) (width 0.2) (layer "F.Cu") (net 8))
 (segment (start 108.067176 105.426) (end 118.014 105.426) (width 0.2) (layer "F.Cu") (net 8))
 (segment (start 119.464 104.926) (end 119.5 104.89) (width 0.2) (layer "F.Cu") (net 8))
 (segment (start 118.014 105.426) (end 118.55 104.89) (width 0.2) (layer "F.Cu") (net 8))
 (segment (start 120.551 97.371) (end 120.45 97.27) (width 0.2) (layer "F.Cu") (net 2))
 (segment (start 110.8 100.8) (end 114.33 97.27) (width 0.2) (layer "F.Cu") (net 2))
 (segment (start 118.449 96.751) (end 118.968 97.27) (width 0.2) (layer "F.Cu") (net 2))
 (segment (start 120.45 97.27) (end 119.5 97.27) (width 0.2) (layer "F.Cu") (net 2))
 (segment (start 118.449 95.249) (end 118.449 96.751) (width 0.2) (layer "F.Cu") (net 2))
 (segment (start 149.025 108.3) (end 149.025 101.99828) (width 0.2) (layer "F.Cu") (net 2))
 (segment (start 142.249 95.249) (end 118.449 95.249) (width 0.2) (layer "F.Cu") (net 2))
 (segment (start 133.924 123.826) (end 129.014 123.826) (width 0.2) (layer "F.Cu") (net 2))
 (segment (start 129.014 123.826) (end 120.551 115.363) (width 0.2) (layer "F.Cu") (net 2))
 (segment (start 120.551 115.363) (end 120.551 97.371) (width 0.2) (layer "F.Cu") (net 2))
 (segment (start 118.968 97.27) (end 119.5 97.27) (width 0.2) (layer "F.Cu") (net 2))
 (segment (start 134.5 123.25) (end 133.924 123.826) (width 0.2) (layer "F.Cu") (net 2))
 (segment (start 142.27572 95.249) (end 118.449 95.249) (width 0.2) (layer "F.Cu") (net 2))
 (segment (start 149.025 101.99828) (end 142.27572 95.249) (width 0.2) (layer "F.Cu") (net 2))
 (segment (start 114.33 97.27) (end 119.5 97.27) (width 0.2) (layer "F.Cu") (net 2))
 (segment (start 145 98) (end 142.249 95.249) (width 0.2) (layer "F.Cu") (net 2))
 (segment (start 149.025 110.3) (end 137.33 110.3) (width 0.2) (layer "F.Cu") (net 26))
 (segment (start 137.33 110.3) (end 137 109.97) (width 0.2) (layer "F.Cu") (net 26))
 (segment (start 137.532 109.97) (end 137 109.97) (width 0.2) (layer "F.Cu") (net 26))
 (segment (start 148.250001 109.3) (end 147.650001 108.7) (width 0.2) (layer "F.Cu") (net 27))
 (segment (start 149.025 109.3) (end 148.250001 109.3) (width 0.2) (layer "F.Cu") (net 27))
 (segment (start 147.650001 108.7) (end 137 108.7) (width 0.2) (layer "F.Cu") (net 27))
 (segment (start 136.468 108.7) (end 137 108.7) (width 0.2) (layer "F.Cu") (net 27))
 (segment (start 106.473 108.6661) (end 122.0339 124.227) (width 0.2) (layer "F.Cu") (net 1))
 (segment (start 126.045 104.865) (end 122.54 108.37) (width 0.2) (layer "F.Cu") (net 1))
 (segment (start 122.54 108.37) (end 122.54 113.76) (width 0.2) (layer "F.Cu") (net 1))
 (segment (start 134.5 120.75) (end 134.7 120.75) (width 0.2) (layer "F.Cu") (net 1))
 (segment (start 135.276 113.264) (end 134.721 112.709) (width 0.2) (layer "F.Cu") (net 1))
 (segment (start 122.0339 124.227) (end 134.875 124.227) (width 0.2) (layer "F.Cu") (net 1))
 (segment (start 120.23 96) (end 119.5 96) (width 0.2) (layer "F.Cu") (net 1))
 (segment (start 106.473 101.668176) (end 106.473 108.6661) (width 0.2) (layer "F.Cu") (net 1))
 (segment (start 126.045 101.815) (end 120.23 96) (width 0.2) (layer "F.Cu") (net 1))
 (segment (start 134.721 112.709) (end 123.059 112.709) (width 0.2) (layer "F.Cu") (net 1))
 (segment (start 149.025 111.3) (end 140.012 111.3) (width 0.2) (layer "F.Cu") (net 1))
 (segment (start 140.012 115.438) (end 140.012 111.3) (width 0.2) (layer "F.Cu") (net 1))
 (segment (start 134.91 96) (end 137 96) (width 0.2) (layer "F.Cu") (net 1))
 (segment (start 123.059 112.709) (end 122.54 113.228) (width 0.2) (layer "F.Cu") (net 1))
 (segment (start 108.3 100.8) (end 107.341176 100.8) (width 0.2) (layer "F.Cu") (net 1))
 (segment (start 134.7 120.75) (end 140.012 115.438) (width 0.2) (layer "F.Cu") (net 1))
 (segment (start 107.341176 100.8) (end 106.473 101.668176) (width 0.2) (layer "F.Cu") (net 1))
 (segment (start 134.875 124.227) (end 135.276 123.826) (width 0.2) (layer "F.Cu") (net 1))
 (segment (start 140.012 111.3) (end 137.552 113.76) (width 0.2) (layer "F.Cu") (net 1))
 (segment (start 135.772 113.76) (end 134.721 112.709) (width 0.2) (layer "F.Cu") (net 1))
 (segment (start 137.552 113.76) (end 135.772 113.76) (width 0.2) (layer "F.Cu") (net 1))
 (segment (start 135.276 123.826) (end 135.276 113.264) (width 0.2) (layer "F.Cu") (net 1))
 (segment (start 122.54 113.228) (end 122.54 113.76) (width 0.2) (layer "F.Cu") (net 1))
 (segment (start 129.095 101.815) (end 134.91 96) (width 0.2) (layer "F.Cu") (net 1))
 (segment (start 145 102) (end 129.6725 102) (width 0.2) (layer "B.Cu") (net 1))
 (segment (start 129.6725 102) (end 129.095 102.5775) (width 0.2) (layer "B.Cu") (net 1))
 (segment (start 145 100) (end 144.5 100) (width 0.2) (layer "F.Cu") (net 34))
 (segment (start 144.5 100) (end 144.31 99.81) (width 0.2) (layer "F.Cu") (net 34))
 (segment (start 144.31 99.81) (end 137 99.81) (width 0.2) (layer "F.Cu") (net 34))
 (segment (start 145 101) (end 144.5 101) (width 0.2) (layer "F.Cu") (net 33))
 (segment (start 144.42 101.08) (end 137 101.08) (width 0.2) (layer "F.Cu") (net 33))
 (segment (start 144.5 101) (end 144.42 101.08) (width 0.2) (layer "F.Cu") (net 33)))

